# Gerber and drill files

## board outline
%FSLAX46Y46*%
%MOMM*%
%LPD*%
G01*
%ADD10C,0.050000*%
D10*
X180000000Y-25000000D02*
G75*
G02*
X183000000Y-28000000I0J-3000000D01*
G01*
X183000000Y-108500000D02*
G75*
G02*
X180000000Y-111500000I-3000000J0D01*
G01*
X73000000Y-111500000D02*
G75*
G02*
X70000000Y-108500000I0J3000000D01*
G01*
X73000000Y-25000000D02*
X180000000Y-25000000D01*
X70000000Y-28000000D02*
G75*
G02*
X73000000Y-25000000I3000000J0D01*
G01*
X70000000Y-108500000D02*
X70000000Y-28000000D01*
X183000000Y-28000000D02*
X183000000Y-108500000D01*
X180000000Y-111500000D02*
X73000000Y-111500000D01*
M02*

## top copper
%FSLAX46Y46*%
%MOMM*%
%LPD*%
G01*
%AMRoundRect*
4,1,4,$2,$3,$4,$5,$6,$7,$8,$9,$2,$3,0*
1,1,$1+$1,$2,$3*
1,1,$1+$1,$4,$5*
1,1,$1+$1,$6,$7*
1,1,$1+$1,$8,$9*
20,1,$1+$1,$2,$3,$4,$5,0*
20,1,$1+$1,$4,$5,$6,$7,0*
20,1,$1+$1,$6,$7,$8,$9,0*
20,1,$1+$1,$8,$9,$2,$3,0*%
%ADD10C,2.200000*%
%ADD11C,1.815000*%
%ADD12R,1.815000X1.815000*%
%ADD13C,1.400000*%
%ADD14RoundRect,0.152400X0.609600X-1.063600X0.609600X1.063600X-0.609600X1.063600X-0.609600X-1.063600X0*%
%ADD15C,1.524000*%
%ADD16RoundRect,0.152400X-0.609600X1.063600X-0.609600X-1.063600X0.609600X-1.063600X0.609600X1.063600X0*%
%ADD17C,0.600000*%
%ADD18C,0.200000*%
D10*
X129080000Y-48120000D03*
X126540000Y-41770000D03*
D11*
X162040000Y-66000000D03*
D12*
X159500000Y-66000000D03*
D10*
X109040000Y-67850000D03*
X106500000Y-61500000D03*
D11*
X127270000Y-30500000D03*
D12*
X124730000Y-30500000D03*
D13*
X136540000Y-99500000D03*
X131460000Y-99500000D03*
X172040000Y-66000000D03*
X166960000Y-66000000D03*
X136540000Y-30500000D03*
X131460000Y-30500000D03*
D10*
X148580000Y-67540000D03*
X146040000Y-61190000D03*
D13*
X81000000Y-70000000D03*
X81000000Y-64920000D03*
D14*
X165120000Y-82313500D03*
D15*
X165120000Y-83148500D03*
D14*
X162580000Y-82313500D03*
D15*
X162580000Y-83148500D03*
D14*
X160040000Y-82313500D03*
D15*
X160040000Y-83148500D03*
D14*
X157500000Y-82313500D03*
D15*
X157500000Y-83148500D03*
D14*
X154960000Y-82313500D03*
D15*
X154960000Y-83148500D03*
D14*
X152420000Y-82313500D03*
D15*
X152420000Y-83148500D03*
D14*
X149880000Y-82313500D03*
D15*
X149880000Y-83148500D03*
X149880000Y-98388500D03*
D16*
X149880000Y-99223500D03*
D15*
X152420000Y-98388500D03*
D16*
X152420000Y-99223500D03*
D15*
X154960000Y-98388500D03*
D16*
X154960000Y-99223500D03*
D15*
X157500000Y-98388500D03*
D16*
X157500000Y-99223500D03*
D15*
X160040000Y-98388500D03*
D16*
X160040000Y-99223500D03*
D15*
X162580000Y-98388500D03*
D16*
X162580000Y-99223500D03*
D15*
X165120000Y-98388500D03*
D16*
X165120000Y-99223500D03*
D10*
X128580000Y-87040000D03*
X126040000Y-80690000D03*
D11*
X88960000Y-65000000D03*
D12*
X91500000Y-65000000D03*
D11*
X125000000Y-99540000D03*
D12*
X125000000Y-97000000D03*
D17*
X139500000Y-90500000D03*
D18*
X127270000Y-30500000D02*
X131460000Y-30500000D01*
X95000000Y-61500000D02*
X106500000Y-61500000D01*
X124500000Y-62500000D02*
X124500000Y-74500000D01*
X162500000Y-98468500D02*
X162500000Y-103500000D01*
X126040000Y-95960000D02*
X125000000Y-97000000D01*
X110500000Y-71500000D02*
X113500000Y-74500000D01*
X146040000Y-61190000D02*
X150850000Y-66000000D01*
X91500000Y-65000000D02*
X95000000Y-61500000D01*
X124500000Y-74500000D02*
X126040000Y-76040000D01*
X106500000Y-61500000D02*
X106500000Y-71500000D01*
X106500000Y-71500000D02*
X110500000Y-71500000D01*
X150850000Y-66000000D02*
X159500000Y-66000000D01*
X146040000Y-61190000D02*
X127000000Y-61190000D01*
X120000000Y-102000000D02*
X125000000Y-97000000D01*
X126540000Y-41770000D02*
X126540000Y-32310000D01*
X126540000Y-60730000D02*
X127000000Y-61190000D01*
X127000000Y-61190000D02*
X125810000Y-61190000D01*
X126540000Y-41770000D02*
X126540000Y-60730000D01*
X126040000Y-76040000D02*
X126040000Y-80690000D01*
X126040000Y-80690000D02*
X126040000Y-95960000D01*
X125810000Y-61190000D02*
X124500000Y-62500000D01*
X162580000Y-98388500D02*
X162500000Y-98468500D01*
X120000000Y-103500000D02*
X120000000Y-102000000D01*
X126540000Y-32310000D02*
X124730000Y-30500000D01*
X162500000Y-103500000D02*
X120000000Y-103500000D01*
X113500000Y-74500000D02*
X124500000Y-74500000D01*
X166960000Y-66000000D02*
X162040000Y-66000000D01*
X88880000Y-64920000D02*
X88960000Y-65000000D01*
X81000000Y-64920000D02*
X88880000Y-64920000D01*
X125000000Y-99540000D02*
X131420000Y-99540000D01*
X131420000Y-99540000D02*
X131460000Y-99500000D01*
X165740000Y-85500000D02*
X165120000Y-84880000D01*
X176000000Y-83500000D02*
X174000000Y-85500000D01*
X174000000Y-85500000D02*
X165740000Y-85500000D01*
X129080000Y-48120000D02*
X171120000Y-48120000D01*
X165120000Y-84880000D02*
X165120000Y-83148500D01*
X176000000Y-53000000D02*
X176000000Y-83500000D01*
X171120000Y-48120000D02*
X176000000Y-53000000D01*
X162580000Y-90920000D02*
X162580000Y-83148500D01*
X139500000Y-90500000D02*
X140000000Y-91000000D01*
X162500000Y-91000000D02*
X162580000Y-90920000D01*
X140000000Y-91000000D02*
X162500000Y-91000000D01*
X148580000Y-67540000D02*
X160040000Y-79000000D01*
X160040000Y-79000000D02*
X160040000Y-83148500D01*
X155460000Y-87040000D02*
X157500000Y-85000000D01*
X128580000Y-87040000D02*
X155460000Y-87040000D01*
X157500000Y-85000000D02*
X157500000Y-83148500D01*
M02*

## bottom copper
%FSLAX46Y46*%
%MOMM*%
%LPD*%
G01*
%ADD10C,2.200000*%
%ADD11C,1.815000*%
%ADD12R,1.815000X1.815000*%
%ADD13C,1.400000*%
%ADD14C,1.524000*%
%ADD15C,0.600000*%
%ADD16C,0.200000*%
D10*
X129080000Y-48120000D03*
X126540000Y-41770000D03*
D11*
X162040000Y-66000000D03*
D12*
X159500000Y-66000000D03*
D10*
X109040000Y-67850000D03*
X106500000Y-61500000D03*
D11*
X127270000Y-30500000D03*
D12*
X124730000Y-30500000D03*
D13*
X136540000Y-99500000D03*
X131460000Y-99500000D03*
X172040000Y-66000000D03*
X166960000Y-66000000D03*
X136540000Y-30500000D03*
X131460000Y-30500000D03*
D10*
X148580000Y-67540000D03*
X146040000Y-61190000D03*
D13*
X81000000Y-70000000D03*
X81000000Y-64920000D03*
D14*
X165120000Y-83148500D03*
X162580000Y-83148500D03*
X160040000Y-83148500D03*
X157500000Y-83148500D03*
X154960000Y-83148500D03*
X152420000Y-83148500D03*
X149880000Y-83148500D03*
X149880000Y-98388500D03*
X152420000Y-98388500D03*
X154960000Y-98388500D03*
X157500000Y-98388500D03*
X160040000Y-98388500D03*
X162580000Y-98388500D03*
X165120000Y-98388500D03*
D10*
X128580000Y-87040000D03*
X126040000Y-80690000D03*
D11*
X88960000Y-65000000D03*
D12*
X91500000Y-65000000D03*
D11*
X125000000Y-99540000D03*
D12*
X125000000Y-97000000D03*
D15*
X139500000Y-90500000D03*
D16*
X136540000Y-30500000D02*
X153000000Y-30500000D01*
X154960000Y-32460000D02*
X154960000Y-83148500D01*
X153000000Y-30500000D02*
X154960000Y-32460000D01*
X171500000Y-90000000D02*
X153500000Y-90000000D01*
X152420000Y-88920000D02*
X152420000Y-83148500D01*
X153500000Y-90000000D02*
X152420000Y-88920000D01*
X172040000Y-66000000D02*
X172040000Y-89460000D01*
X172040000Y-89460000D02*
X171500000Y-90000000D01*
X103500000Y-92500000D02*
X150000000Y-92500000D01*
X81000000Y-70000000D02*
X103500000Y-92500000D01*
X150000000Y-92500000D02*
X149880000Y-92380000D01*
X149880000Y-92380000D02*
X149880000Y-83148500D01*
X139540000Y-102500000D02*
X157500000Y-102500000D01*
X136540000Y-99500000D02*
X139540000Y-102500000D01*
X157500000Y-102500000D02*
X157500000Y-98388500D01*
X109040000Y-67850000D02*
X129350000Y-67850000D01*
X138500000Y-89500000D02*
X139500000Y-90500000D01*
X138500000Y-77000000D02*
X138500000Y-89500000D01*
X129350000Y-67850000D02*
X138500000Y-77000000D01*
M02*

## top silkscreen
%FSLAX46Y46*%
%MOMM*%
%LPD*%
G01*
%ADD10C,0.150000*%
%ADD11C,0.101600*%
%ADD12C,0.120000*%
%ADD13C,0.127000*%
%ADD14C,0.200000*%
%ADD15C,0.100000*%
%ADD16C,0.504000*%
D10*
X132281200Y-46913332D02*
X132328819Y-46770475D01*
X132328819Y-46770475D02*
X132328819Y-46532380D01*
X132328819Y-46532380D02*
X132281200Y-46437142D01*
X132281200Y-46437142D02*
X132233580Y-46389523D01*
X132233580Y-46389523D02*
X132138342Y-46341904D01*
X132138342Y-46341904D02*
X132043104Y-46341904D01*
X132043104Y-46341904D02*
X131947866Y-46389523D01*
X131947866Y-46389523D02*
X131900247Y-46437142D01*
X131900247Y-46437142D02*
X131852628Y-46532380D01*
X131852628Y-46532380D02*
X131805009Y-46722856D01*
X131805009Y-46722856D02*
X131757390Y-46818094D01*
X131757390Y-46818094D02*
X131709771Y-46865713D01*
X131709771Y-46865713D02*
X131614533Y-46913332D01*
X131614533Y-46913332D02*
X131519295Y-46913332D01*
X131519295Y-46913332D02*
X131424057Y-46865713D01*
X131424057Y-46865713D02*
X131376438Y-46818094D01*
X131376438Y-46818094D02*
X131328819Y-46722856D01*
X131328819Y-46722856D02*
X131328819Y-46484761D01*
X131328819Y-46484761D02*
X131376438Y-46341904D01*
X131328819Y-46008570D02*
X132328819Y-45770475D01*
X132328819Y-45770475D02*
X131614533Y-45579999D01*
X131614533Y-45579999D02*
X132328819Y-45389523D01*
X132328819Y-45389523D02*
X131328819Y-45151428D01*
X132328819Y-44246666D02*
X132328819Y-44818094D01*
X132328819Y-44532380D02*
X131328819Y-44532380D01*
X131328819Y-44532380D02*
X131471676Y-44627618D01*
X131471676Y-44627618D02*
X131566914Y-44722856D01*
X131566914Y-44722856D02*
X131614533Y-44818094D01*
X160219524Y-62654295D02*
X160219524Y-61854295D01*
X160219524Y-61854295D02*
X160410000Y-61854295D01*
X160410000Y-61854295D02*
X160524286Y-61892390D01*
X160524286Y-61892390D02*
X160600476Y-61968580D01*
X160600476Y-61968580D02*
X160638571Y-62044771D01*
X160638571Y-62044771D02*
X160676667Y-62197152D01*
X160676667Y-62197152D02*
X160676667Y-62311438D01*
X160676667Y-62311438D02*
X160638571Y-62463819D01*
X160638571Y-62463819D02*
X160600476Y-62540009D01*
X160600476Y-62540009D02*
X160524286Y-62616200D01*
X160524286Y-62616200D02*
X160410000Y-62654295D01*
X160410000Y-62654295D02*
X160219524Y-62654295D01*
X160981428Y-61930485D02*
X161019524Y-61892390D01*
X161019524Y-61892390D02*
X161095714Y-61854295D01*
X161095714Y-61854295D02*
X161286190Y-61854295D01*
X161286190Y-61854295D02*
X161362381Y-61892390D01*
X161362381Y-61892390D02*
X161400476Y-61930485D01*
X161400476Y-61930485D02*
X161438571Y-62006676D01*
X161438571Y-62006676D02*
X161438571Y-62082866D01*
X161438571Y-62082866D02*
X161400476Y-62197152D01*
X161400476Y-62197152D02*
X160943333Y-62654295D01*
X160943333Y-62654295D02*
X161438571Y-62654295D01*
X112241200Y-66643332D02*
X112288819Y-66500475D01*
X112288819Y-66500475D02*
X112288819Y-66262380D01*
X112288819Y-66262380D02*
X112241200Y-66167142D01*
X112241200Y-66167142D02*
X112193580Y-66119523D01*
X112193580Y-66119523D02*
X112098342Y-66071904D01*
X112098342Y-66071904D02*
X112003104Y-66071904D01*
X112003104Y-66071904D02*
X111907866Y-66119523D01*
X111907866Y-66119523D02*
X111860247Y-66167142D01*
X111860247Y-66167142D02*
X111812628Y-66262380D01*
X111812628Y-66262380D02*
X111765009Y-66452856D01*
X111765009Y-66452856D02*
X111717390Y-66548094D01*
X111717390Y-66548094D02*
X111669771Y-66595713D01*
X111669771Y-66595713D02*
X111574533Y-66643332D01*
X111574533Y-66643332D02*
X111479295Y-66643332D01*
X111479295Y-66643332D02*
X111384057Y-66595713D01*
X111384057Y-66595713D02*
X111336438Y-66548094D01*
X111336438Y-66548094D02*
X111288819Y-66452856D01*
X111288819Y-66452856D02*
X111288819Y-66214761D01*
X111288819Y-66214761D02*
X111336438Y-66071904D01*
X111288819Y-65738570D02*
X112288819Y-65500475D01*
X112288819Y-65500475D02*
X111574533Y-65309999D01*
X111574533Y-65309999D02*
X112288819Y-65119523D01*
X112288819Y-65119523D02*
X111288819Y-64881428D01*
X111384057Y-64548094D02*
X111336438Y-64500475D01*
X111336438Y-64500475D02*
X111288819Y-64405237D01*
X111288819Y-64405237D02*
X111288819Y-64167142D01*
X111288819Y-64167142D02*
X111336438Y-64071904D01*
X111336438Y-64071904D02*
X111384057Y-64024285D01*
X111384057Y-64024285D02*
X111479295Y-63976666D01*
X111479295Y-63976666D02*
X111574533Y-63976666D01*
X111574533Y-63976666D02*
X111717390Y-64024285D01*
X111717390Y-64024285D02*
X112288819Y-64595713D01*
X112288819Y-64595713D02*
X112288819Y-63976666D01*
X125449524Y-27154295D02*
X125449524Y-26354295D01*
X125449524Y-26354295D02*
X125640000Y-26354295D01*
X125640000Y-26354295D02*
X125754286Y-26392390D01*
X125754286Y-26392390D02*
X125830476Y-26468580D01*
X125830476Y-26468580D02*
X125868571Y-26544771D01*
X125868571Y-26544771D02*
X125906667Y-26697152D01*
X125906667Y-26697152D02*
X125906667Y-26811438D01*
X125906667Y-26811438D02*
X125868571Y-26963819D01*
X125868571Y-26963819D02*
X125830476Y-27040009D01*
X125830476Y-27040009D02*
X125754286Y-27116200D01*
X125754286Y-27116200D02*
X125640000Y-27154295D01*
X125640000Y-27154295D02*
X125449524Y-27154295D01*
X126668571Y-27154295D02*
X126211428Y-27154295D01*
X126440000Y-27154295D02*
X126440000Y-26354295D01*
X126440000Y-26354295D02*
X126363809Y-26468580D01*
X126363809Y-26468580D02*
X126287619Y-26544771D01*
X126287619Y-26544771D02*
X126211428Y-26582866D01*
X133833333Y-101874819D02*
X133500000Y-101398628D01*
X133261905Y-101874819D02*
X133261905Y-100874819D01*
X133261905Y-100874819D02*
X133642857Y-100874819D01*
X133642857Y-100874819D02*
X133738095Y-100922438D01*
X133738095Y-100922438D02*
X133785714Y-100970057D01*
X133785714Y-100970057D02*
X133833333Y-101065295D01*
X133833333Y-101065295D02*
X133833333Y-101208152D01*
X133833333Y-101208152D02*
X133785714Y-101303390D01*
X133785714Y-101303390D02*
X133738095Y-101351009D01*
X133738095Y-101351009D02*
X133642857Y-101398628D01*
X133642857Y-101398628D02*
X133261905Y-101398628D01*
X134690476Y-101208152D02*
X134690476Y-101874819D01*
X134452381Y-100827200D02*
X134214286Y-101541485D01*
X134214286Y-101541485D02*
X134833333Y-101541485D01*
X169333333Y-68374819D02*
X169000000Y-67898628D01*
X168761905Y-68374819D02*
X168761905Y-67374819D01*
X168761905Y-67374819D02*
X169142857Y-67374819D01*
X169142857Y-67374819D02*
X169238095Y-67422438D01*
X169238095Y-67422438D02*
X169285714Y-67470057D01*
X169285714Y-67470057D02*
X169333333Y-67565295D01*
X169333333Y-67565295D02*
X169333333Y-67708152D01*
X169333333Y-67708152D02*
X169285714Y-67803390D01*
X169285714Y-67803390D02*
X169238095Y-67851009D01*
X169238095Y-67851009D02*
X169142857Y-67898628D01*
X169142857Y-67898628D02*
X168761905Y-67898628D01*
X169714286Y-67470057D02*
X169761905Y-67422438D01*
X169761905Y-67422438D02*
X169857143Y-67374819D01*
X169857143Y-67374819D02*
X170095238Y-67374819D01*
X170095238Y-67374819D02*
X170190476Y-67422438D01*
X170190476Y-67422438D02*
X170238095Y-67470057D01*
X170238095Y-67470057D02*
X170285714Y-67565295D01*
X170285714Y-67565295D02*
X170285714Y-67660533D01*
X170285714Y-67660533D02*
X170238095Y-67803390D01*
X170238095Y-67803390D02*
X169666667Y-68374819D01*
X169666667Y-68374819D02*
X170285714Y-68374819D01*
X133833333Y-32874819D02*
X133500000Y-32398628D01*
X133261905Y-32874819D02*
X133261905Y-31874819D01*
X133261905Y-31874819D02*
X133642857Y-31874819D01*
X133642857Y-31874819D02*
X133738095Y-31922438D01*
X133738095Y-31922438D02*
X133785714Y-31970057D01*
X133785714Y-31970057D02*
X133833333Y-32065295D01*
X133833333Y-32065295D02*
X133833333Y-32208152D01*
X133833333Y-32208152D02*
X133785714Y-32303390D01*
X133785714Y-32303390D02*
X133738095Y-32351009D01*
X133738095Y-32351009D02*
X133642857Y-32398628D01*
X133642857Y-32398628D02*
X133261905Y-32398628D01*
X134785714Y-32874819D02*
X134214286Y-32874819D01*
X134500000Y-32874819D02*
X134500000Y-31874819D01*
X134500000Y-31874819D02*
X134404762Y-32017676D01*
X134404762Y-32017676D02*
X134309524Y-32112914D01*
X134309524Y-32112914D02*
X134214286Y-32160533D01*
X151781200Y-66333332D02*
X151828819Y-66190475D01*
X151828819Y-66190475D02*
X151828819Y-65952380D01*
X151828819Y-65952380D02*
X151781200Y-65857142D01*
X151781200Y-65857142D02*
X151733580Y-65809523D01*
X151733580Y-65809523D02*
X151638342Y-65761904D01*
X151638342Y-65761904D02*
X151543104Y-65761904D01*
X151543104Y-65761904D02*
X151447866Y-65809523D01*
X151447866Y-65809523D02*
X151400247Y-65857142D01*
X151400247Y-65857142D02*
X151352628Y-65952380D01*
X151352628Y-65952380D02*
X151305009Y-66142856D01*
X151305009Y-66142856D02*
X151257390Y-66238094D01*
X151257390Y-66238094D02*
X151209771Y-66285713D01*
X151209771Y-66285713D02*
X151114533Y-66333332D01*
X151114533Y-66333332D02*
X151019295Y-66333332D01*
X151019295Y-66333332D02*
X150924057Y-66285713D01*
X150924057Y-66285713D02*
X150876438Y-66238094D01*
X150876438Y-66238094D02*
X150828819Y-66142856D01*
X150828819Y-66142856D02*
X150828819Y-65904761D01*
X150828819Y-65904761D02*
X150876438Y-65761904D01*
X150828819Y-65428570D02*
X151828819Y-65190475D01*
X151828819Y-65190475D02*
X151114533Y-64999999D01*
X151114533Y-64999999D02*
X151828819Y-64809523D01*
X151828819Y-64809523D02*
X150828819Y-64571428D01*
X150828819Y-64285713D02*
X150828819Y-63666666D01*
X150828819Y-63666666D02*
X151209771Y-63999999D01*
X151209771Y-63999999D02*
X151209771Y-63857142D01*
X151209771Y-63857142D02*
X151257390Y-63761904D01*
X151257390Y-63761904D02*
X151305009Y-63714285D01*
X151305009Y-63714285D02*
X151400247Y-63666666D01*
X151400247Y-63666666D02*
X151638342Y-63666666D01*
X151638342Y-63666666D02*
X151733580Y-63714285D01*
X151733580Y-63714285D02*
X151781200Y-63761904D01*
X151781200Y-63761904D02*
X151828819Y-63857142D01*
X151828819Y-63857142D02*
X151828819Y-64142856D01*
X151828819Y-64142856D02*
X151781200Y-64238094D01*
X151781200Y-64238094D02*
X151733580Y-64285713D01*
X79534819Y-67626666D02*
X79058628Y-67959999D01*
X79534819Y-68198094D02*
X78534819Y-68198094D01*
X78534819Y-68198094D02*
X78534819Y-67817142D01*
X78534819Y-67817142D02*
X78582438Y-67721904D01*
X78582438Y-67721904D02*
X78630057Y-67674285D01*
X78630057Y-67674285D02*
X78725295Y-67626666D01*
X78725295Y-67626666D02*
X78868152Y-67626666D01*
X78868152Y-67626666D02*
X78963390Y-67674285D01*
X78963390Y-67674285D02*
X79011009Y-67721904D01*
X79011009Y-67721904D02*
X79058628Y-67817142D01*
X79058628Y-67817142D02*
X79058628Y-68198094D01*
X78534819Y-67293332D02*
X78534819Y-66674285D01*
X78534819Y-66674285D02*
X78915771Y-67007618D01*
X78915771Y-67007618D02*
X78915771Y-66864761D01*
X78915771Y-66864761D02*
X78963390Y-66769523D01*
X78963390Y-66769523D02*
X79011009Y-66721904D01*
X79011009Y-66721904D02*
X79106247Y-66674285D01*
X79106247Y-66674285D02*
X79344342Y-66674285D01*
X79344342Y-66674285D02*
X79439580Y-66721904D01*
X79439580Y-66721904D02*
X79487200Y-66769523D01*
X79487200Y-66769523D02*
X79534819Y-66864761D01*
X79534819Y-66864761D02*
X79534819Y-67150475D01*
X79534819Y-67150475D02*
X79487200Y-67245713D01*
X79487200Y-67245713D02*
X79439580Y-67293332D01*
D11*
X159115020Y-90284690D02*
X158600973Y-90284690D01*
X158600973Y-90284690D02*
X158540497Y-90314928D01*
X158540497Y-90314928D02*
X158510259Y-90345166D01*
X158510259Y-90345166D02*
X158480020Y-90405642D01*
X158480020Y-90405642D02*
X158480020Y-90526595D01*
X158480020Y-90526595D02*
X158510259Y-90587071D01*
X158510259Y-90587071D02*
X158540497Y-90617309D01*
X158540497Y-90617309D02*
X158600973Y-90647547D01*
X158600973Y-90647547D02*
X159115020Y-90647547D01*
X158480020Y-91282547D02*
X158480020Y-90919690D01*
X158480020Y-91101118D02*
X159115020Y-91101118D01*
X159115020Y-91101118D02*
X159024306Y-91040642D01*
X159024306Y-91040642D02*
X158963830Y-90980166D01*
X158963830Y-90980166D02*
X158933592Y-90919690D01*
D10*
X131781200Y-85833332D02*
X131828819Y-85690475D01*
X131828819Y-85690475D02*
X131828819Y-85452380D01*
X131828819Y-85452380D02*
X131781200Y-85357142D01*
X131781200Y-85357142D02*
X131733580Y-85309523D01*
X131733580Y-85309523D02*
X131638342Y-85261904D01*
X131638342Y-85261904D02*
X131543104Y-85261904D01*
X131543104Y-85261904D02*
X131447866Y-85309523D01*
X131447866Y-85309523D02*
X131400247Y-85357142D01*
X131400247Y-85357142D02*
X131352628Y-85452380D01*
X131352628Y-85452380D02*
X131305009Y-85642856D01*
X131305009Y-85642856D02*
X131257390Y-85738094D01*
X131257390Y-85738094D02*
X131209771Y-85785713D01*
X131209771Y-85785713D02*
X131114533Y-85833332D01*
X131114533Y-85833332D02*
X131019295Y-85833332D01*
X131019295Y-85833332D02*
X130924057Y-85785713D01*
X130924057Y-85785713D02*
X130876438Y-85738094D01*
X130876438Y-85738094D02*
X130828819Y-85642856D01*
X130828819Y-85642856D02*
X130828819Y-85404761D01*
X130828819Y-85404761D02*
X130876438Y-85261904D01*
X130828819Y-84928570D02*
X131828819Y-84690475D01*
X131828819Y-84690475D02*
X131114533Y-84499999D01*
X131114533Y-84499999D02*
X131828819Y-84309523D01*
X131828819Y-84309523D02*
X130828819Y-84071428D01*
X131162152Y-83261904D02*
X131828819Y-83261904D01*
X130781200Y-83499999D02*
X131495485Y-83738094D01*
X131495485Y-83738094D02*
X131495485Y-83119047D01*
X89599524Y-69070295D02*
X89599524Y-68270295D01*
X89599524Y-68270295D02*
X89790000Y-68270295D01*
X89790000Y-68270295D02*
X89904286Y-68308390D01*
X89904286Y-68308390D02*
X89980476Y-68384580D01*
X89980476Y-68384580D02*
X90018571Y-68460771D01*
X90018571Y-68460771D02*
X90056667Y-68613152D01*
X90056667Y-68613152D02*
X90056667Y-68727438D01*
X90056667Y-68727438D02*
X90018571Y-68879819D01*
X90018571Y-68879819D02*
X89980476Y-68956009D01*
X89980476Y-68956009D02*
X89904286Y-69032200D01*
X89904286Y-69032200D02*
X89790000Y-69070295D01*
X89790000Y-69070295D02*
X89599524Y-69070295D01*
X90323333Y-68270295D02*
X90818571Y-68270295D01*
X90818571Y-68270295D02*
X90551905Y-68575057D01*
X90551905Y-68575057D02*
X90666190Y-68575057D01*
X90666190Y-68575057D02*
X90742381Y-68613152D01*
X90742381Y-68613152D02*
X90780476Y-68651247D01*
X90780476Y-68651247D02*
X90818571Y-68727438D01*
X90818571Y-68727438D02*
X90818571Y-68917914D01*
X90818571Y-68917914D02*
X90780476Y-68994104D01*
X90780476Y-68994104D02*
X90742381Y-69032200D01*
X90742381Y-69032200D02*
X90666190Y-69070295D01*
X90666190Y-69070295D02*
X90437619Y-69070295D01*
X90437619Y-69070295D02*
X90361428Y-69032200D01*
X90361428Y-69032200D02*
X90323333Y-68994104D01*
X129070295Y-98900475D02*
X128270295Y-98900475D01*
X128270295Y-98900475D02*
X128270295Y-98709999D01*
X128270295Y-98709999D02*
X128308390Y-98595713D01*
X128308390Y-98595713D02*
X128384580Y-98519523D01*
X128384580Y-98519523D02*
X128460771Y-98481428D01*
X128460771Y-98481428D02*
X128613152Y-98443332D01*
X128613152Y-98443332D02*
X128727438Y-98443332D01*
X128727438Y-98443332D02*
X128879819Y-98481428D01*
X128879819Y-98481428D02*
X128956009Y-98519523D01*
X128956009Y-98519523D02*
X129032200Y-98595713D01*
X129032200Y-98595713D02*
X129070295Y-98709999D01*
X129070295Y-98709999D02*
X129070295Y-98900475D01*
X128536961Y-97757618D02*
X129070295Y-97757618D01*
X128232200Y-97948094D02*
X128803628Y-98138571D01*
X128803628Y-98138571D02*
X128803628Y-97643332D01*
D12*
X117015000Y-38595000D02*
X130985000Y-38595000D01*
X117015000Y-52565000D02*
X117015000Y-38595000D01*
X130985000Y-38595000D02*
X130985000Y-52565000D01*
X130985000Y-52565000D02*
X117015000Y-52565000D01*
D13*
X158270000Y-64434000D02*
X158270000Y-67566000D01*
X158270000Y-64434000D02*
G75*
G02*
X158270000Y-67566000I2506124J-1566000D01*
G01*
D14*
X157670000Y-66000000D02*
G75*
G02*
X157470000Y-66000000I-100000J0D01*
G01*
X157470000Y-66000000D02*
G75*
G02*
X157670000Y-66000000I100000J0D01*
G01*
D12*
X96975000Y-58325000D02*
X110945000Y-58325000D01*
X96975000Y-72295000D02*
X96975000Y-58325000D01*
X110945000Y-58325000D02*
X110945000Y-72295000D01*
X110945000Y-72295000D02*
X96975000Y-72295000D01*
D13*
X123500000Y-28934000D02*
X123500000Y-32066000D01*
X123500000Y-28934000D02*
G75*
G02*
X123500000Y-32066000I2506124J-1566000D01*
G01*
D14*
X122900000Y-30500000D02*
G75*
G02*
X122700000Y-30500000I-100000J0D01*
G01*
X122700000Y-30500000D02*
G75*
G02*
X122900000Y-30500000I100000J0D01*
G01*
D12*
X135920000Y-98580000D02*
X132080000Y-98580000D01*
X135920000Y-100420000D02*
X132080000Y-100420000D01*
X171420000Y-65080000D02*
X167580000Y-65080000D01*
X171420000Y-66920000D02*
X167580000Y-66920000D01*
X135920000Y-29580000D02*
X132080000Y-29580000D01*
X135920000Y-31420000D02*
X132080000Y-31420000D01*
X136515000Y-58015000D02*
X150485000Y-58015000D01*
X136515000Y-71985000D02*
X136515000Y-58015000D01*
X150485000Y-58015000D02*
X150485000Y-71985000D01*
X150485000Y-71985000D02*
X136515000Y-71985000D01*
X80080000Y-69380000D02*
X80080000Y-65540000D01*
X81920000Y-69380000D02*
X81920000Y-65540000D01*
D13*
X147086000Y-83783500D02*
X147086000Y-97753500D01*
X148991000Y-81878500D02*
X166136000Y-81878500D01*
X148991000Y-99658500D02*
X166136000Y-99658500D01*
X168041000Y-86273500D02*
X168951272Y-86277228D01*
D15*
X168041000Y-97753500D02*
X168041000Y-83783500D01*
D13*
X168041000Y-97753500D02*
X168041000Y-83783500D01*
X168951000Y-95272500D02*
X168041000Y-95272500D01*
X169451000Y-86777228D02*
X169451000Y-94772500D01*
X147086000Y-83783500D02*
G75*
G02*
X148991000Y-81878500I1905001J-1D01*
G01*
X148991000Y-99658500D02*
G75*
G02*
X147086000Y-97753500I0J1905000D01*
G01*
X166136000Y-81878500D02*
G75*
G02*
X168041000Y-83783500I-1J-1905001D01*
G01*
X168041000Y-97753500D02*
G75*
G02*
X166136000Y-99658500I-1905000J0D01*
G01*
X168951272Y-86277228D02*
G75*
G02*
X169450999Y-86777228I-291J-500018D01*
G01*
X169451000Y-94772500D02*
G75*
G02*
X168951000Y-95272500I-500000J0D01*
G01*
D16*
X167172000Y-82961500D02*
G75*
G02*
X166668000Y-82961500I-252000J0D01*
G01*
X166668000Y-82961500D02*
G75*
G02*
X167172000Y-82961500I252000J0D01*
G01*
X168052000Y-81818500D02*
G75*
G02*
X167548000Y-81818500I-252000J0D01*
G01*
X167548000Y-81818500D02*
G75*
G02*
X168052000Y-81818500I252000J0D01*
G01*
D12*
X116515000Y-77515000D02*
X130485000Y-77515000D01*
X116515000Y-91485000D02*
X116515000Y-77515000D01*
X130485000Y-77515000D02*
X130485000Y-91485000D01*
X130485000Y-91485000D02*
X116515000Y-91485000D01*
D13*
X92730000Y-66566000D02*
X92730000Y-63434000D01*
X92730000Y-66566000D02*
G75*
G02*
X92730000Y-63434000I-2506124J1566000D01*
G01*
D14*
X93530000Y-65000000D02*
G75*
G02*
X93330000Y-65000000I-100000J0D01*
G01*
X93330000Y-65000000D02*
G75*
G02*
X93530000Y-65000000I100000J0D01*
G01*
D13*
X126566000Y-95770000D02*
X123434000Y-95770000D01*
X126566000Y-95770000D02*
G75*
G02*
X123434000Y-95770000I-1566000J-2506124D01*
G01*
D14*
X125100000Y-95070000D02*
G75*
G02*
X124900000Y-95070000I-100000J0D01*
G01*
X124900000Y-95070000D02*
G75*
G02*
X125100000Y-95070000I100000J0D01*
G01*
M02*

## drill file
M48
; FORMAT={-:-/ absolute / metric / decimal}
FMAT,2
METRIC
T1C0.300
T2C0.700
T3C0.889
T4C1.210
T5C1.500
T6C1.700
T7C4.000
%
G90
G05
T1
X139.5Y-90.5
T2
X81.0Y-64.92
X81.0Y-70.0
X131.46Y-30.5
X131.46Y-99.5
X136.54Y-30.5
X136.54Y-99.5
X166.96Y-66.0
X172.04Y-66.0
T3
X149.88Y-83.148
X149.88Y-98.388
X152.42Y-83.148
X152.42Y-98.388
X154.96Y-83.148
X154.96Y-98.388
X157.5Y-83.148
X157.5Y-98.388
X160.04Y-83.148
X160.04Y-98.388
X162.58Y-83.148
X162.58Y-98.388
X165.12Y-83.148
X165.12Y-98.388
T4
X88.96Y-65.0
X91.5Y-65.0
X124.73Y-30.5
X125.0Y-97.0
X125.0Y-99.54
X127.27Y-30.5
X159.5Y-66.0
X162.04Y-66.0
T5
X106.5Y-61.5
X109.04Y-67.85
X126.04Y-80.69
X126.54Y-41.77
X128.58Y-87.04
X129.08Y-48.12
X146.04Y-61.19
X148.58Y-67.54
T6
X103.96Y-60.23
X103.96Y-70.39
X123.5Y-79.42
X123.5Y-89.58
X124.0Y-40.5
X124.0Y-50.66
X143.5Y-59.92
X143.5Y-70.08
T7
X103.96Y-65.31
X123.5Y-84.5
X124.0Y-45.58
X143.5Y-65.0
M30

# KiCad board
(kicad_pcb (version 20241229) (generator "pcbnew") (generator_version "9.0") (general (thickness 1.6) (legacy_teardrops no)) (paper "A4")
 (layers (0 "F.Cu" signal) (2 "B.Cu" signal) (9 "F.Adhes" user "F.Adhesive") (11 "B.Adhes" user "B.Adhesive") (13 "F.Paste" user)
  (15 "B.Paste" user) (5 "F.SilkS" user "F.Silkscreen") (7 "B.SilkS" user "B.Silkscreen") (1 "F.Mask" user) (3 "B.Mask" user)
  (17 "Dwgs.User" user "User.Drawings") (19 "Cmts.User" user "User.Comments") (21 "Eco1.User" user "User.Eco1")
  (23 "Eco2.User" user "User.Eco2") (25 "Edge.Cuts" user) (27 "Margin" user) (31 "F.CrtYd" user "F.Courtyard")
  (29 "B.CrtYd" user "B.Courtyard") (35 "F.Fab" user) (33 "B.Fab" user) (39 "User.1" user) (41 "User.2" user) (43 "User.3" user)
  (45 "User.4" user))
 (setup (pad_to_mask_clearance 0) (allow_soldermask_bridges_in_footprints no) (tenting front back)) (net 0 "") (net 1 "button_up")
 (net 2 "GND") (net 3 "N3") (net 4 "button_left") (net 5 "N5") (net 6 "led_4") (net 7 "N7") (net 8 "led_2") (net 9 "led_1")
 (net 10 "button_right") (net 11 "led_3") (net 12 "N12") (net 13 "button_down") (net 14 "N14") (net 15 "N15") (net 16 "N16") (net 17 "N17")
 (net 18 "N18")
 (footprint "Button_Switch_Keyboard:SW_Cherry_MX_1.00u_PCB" (layer "F.Cu") (at 129.08 48.12 -90)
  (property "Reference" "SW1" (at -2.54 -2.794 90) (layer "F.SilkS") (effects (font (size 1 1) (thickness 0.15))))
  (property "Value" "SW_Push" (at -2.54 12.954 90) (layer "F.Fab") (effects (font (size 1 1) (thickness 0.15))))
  (fp_line (start -9.525 12.065) (end -9.525 -1.905) (stroke (width 0.12) (type solid)) (layer "F.SilkS"))
  (fp_line (start 4.445 12.065) (end -9.525 12.065) (stroke (width 0.12) (type solid)) (layer "F.SilkS"))
  (fp_line (start -9.525 -1.905) (end 4.445 -1.905) (stroke (width 0.12) (type solid)) (layer "F.SilkS"))
  (fp_line (start 4.445 -1.905) (end 4.445 12.065) (stroke (width 0.12) (type solid)) (layer "F.SilkS"))
  (pad "" np_thru_hole circle (at -7.62 5.08 270) (size 1.7 1.7) (drill 1.7) (layers "*.Cu" "*.Mask"))
  (pad "" np_thru_hole circle (at -2.54 5.08 270) (size 4 4) (drill 4) (layers "*.Cu" "*.Mask"))
  (pad "" np_thru_hole circle (at 2.54 5.08 270) (size 1.7 1.7) (drill 1.7) (layers "*.Cu" "*.Mask"))
  (pad "1" thru_hole circle (at 0 0 270) (size 2.2 2.2) (drill 1.5) (layers "*.Cu" "*.Mask") (remove_unused_layers no) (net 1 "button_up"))
  (pad "2" thru_hole circle (at -6.35 2.54 270) (size 2.2 2.2) (drill 1.5) (layers "*.Cu" "*.Mask") (remove_unused_layers no) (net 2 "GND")))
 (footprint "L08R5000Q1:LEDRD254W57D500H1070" (layer "F.Cu") (at 160.77 66)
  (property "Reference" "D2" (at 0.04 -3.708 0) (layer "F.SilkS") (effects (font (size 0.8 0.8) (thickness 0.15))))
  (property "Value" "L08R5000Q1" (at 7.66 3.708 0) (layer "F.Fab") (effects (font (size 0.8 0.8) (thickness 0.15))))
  (fp_line (start -2.5 -1.566) (end -2.5 1.566) (stroke (width 0.127) (type solid)) (layer "F.SilkS"))
  (fp_arc (start -2.5 -1.566) (mid 2.961291 0) (end -2.5 1.566) (stroke (width 0.127) (type solid)) (layer "F.SilkS"))
  (fp_circle (center -3.2 0) (end -3.1 0) (stroke (width 0.2) (type solid)) (fill no) (layer "F.SilkS"))
  (pad "A" thru_hole circle (at 1.27 0) (size 1.815 1.815) (drill 1.21) (layers "*.Cu" "*.Mask") (remove_unused_layers no) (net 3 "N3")
   (solder_mask_margin 0.102))
  (pad "C" thru_hole rect (at -1.27 0) (size 1.815 1.815) (drill 1.21) (layers "*.Cu" "*.Mask") (remove_unused_layers no) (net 2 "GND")
   (solder_mask_margin 0.102)))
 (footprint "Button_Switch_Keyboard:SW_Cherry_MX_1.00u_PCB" (layer "F.Cu") (at 109.04 67.85 -90)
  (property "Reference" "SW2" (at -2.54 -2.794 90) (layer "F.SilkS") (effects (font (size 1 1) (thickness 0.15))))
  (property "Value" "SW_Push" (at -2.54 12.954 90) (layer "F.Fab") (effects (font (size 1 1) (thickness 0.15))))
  (fp_line (start -9.525 12.065) (end -9.525 -1.905) (stroke (width 0.12) (type solid)) (layer "F.SilkS"))
  (fp_line (start 4.445 12.065) (end -9.525 12.065) (stroke (width 0.12) (type solid)) (layer "F.SilkS"))
  (fp_line (start -9.525 -1.905) (end 4.445 -1.905) (stroke (width 0.12) (type solid)) (layer "F.SilkS"))
  (fp_line (start 4.445 -1.905) (end 4.445 12.065) (stroke (width 0.12) (type solid)) (layer "F.SilkS"))
  (pad "" np_thru_hole circle (at -7.62 5.08 270) (size 1.7 1.7) (drill 1.7) (layers "*.Cu" "*.Mask"))
  (pad "" np_thru_hole circle (at -2.54 5.08 270) (size 4 4) (drill 4) (layers "*.Cu" "*.Mask"))
  (pad "" np_thru_hole circle (at 2.54 5.08 270) (size 1.7 1.7) (drill 1.7) (layers "*.Cu" "*.Mask"))
  (pad "1" thru_hole circle (at 0 0 270) (size 2.2 2.2) (drill 1.5) (layers "*.Cu" "*.Mask") (remove_unused_layers no) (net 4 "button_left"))
  (pad "2" thru_hole circle (at -6.35 2.54 270) (size 2.2 2.2) (drill 1.5) (layers "*.Cu" "*.Mask") (remove_unused_layers no) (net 2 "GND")))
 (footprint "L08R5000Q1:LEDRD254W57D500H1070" (layer "F.Cu") (at 126 30.5)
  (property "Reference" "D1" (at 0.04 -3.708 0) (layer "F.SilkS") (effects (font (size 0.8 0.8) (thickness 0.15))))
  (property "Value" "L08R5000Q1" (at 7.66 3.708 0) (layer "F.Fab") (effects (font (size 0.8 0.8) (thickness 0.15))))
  (fp_line (start -2.5 -1.566) (end -2.5 1.566) (stroke (width 0.127) (type solid)) (layer "F.SilkS"))
  (fp_arc (start -2.5 -1.566) (mid 2.961291 0) (end -2.5 1.566) (stroke (width 0.127) (type solid)) (layer "F.SilkS"))
  (fp_circle (center -3.2 0) (end -3.1 0) (stroke (width 0.2) (type solid)) (fill no) (layer "F.SilkS"))
  (pad "A" thru_hole circle (at 1.27 0) (size 1.815 1.815) (drill 1.21) (layers "*.Cu" "*.Mask") (remove_unused_layers no) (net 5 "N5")
   (solder_mask_margin 0.102))
  (pad "C" thru_hole rect (at -1.27 0) (size 1.815 1.815) (drill 1.21) (layers "*.Cu" "*.Mask") (remove_unused_layers no) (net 2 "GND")
   (solder_mask_margin 0.102)))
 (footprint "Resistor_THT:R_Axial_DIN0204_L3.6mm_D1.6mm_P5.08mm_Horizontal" (layer "F.Cu") (at 136.54 99.5 180)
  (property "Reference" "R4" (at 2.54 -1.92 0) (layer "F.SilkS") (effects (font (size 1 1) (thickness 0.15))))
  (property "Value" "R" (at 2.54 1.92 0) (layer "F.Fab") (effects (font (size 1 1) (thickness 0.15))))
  (fp_line (start 0.62 0.92) (end 4.46 0.92) (stroke (width 0.12) (type solid)) (layer "F.SilkS"))
  (fp_line (start 0.62 -0.92) (end 4.46 -0.92) (stroke (width 0.12) (type solid)) (layer "F.SilkS"))
  (pad "1" thru_hole circle (at 0 0 180) (size 1.4 1.4) (drill 0.7) (layers "*.Cu" "*.Mask") (remove_unused_layers no) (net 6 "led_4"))
  (pad "2" thru_hole circle (at 5.08 0 180) (size 1.4 1.4) (drill 0.7) (layers "*.Cu" "*.Mask") (remove_unused_layers no) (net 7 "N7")))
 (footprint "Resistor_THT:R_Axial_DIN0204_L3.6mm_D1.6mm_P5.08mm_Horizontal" (layer "F.Cu") (at 172.04 66 180)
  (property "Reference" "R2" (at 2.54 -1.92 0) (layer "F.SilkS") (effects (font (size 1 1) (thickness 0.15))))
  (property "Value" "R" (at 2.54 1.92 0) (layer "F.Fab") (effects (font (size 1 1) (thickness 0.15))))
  (fp_line (start 0.62 0.92) (end 4.46 0.92) (stroke (width 0.12) (type solid)) (layer "F.SilkS"))
  (fp_line (start 0.62 -0.92) (end 4.46 -0.92) (stroke (width 0.12) (type solid)) (layer "F.SilkS"))
  (pad "1" thru_hole circle (at 0 0 180) (size 1.4 1.4) (drill 0.7) (layers "*.Cu" "*.Mask") (remove_unused_layers no) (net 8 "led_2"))
  (pad "2" thru_hole circle (at 5.08 0 180) (size 1.4 1.4) (drill 0.7) (layers "*.Cu" "*.Mask") (remove_unused_layers no) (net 3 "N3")))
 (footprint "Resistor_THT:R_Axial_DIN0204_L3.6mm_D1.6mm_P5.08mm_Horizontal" (layer "F.Cu") (at 136.54 30.5 180)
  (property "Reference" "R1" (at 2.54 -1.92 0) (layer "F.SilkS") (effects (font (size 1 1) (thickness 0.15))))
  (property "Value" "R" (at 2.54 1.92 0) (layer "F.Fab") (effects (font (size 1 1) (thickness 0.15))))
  (fp_line (start 0.62 0.92) (end 4.46 0.92) (stroke (width 0.12) (type solid)) (layer "F.SilkS"))
  (fp_line (start 0.62 -0.92) (end 4.46 -0.92) (stroke (width 0.12) (type solid)) (layer "F.SilkS"))
  (pad "1" thru_hole circle (at 0 0 180) (size 1.4 1.4) (drill 0.7) (layers "*.Cu" "*.Mask") (remove_unused_layers no) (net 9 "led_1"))
  (pad "2" thru_hole circle (at 5.08 0 180) (size 1.4 1.4) (drill 0.7) (layers "*.Cu" "*.Mask") (remove_unused_layers no) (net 5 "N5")))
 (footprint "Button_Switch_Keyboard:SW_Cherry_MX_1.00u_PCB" (layer "F.Cu") (at 148.58 67.54 -90)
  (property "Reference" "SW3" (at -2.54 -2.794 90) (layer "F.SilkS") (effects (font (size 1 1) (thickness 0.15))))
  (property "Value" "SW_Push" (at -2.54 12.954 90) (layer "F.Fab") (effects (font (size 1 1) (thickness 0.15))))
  (fp_line (start -9.525 12.065) (end -9.525 -1.905) (stroke (width 0.12) (type solid)) (layer "F.SilkS"))
  (fp_line (start 4.445 12.065) (end -9.525 12.065) (stroke (width 0.12) (type solid)) (layer "F.SilkS"))
  (fp_line (start -9.525 -1.905) (end 4.445 -1.905) (stroke (width 0.12) (type solid)) (layer "F.SilkS"))
  (fp_line (start 4.445 -1.905) (end 4.445 12.065) (stroke (width 0.12) (type solid)) (layer "F.SilkS"))
  (pad "" np_thru_hole circle (at -7.62 5.08 270) (size 1.7 1.7) (drill 1.7) (layers "*.Cu" "*.Mask"))
  (pad "" np_thru_hole circle (at -2.54 5.08 270) (size 4 4) (drill 4) (layers "*.Cu" "*.Mask"))
  (pad "" np_thru_hole circle (at 2.54 5.08 270) (size 1.7 1.7) (drill 1.7) (layers "*.Cu" "*.Mask"))
  (pad "1" thru_hole circle (at 0 0 270) (size 2.2 2.2) (drill 1.5) (layers "*.Cu" "*.Mask") (remove_unused_layers no)
   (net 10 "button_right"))
  (pad "2" thru_hole circle (at -6.35 2.54 270) (size 2.2 2.2) (drill 1.5) (layers "*.Cu" "*.Mask") (remove_unused_layers no) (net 2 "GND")))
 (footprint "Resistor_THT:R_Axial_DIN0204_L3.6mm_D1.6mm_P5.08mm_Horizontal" (layer "F.Cu") (at 81 70 90)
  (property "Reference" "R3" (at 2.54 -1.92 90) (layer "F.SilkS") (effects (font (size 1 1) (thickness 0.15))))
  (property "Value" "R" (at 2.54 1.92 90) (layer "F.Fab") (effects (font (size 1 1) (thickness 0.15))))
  (fp_line (start 0.62 -0.92) (end 4.46 -0.92) (stroke (width 0.12) (type solid)) (layer "F.SilkS"))
  (fp_line (start 0.62 0.92) (end 4.46 0.92) (stroke (width 0.12) (type solid)) (layer "F.SilkS"))
  (pad "1" thru_hole circle (at 0 0 90) (size 1.4 1.4) (drill 0.7) (layers "*.Cu" "*.Mask") (remove_unused_layers no) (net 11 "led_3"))
  (pad "2" thru_hole circle (at 5.08 0 90) (size 1.4 1.4) (drill 0.7) (layers "*.Cu" "*.Mask") (remove_unused_layers no) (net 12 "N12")))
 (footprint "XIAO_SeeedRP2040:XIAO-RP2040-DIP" (layer "F.Cu") (at 157.5 90.7685 -90)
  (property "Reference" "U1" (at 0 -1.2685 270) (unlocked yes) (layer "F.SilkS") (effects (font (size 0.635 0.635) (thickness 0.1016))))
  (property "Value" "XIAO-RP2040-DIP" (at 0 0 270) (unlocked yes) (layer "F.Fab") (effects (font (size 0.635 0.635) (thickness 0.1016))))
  (fp_line (start -6.985 10.414) (end 6.985 10.414) (stroke (width 0.127) (type solid)) (layer "F.SilkS"))
  (fp_line (start -8.89 8.509) (end -8.89 -8.636) (stroke (width 0.127) (type solid)) (layer "F.SilkS"))
  (fp_line (start 8.89 8.509) (end 8.89 -8.636) (stroke (width 0.127) (type solid)) (layer "F.SilkS"))
  (fp_line (start -4.495 -10.541) (end -4.491272 -11.451272) (stroke (width 0.127) (type solid)) (layer "F.SilkS"))
  (fp_line (start 6.985 -10.541) (end -6.985 -10.541) (stroke (width 0.1) (type solid)) (layer "F.SilkS"))
  (fp_line (start 6.985 -10.541) (end -6.985 -10.541) (stroke (width 0.127) (type solid)) (layer "F.SilkS"))
  (fp_line (start 4.504 -11.451) (end 4.504 -10.541) (stroke (width 0.127) (type solid)) (layer "F.SilkS"))
  (fp_line (start -3.991272 -11.951) (end 4.004 -11.951) (stroke (width 0.127) (type solid)) (layer "F.SilkS"))
  (fp_arc (start -6.985 10.414) (mid -8.332038 9.856038) (end -8.89 8.509) (stroke (width 0.127) (type solid)) (layer "F.SilkS"))
  (fp_arc (start 8.89 8.509) (mid 8.332038 9.856038) (end 6.985 10.414) (stroke (width 0.127) (type solid)) (layer "F.SilkS"))
  (fp_arc (start -8.89 -8.636) (mid -8.332038 -9.983038) (end -6.985 -10.541) (stroke (width 0.127) (type solid)) (layer "F.SilkS"))
  (fp_arc (start 6.985 -10.541) (mid 8.332038 -9.983038) (end 8.89 -8.636) (stroke (width 0.127) (type solid)) (layer "F.SilkS"))
  (fp_arc (start -4.491272 -11.451272) (mid -4.344728 -11.80464) (end -3.991272 -11.951) (stroke (width 0.127) (type default))
   (layer "F.SilkS"))
  (fp_arc (start 4.004 -11.951) (mid 4.357553 -11.804553) (end 4.504 -11.451) (stroke (width 0.127) (type default)) (layer "F.SilkS"))
  (fp_circle (center -7.807 -9.42) (end -7.807 -9.674) (stroke (width 0.5) (type solid)) (fill yes) (layer "F.SilkS"))
  (fp_circle (center -8.95 -10.3) (end -8.95 -10.554) (stroke (width 0.5) (type solid)) (fill yes) (layer "F.SilkS"))
  (pad "1" smd roundrect (at -8.455 -7.62 90) (size 2.432 1.524) (layers "F.Cu" "F.Mask") (roundrect_rratio 0.1) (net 1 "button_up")
   (thermal_bridge_angle 45))
  (pad "1" thru_hole circle (at -7.62 -7.62 90) (size 1.524 1.524) (drill 0.889) (layers "*.Cu" "*.Mask") (remove_unused_layers no)
   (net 1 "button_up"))
  (pad "2" smd roundrect (at -8.455 -5.08 90) (size 2.432 1.524) (layers "F.Cu" "F.Mask") (roundrect_rratio 0.1) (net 4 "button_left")
   (thermal_bridge_angle 45))
  (pad "2" thru_hole circle (at -7.62 -5.08 90) (size 1.524 1.524) (drill 0.889) (layers "*.Cu" "*.Mask") (remove_unused_layers no)
   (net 4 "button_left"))
  (pad "3" smd roundrect (at -8.455 -2.54 90) (size 2.432 1.524) (layers "F.Cu" "F.Mask") (roundrect_rratio 0.1) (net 10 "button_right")
   (thermal_bridge_angle 45))
  (pad "3" thru_hole circle (at -7.62 -2.54 90) (size 1.524 1.524) (drill 0.889) (layers "*.Cu" "*.Mask") (remove_unused_layers no)
   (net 10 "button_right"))
  (pad "4" smd roundrect (at -8.455 0 90) (size 2.432 1.524) (layers "F.Cu" "F.Mask") (roundrect_rratio 0.1) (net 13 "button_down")
   (thermal_bridge_angle 45))
  (pad "4" thru_hole circle (at -7.62 0 90) (size 1.524 1.524) (drill 0.889) (layers "*.Cu" "*.Mask") (remove_unused_layers no)
   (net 13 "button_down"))
  (pad "5" smd roundrect (at -8.455 2.54 90) (size 2.432 1.524) (layers "F.Cu" "F.Mask") (roundrect_rratio 0.1) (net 9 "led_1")
   (thermal_bridge_angle 45))
  (pad "5" thru_hole circle (at -7.62 2.54 90) (size 1.524 1.524) (drill 0.889) (layers "*.Cu" "*.Mask") (remove_unused_layers no)
   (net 9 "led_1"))
  (pad "6" smd roundrect (at -8.455 5.08 90) (size 2.432 1.524) (layers "F.Cu" "F.Mask") (roundrect_rratio 0.1) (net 8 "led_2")
   (thermal_bridge_angle 45))
  (pad "6" thru_hole circle (at -7.62 5.08 90) (size 1.524 1.524) (drill 0.889) (layers "*.Cu" "*.Mask") (remove_unused_layers no)
   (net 8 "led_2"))
  (pad "7" smd roundrect (at -8.455 7.62 90) (size 2.432 1.524) (layers "F.Cu" "F.Mask") (roundrect_rratio 0.1) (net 11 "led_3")
   (thermal_bridge_angle 45))
  (pad "7" thru_hole circle (at -7.62 7.62 90) (size 1.524 1.524) (drill 0.889) (layers "*.Cu" "*.Mask") (remove_unused_layers no)
   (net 11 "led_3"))
  (pad "8" thru_hole circle (at 7.62 7.62 270) (size 1.524 1.524) (drill 0.889) (layers "*.Cu" "*.Mask") (remove_unused_layers no)
   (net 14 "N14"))
  (pad "8" smd roundrect (at 8.455 7.62 270) (size 2.432 1.524) (layers "F.Cu" "F.Mask") (roundrect_rratio 0.1) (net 14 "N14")
   (thermal_bridge_angle 45))
  (pad "9" thru_hole circle (at 7.62 5.08 270) (size 1.524 1.524) (drill 0.889) (layers "*.Cu" "*.Mask") (remove_unused_layers no)
   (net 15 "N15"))
  (pad "9" smd roundrect (at 8.455 5.08 270) (size 2.432 1.524) (layers "F.Cu" "F.Mask") (roundrect_rratio 0.1) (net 15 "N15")
   (thermal_bridge_angle 45))
  (pad "10" thru_hole circle (at 7.62 2.54 270) (size 1.524 1.524) (drill 0.889) (layers "*.Cu" "*.Mask") (remove_unused_layers no)
   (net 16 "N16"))
  (pad "10" smd roundrect (at 8.455 2.54 270) (size 2.432 1.524) (layers "F.Cu" "F.Mask") (roundrect_rratio 0.1) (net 16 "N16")
   (thermal_bridge_angle 45))
  (pad "11" thru_hole circle (at 7.62 0 270) (size 1.524 1.524) (drill 0.889) (layers "*.Cu" "*.Mask") (remove_unused_layers no)
   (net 6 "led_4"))
  (pad "11" smd roundrect (at 8.455 0 270) (size 2.432 1.524) (layers "F.Cu" "F.Mask") (roundrect_rratio 0.1) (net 6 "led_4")
   (thermal_bridge_angle 45))
  (pad "12" thru_hole circle (at 7.62 -2.54 270) (size 1.524 1.524) (drill 0.889) (layers "*.Cu" "*.Mask") (remove_unused_layers no)
   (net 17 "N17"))
  (pad "12" smd roundrect (at 8.455 -2.54 270) (size 2.432 1.524) (layers "F.Cu" "F.Mask") (roundrect_rratio 0.1) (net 17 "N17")
   (thermal_bridge_angle 45))
  (pad "13" thru_hole circle (at 7.62 -5.08 270) (size 1.524 1.524) (drill 0.889) (layers "*.Cu" "*.Mask") (remove_unused_layers no)
   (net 2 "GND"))
  (pad "13" smd roundrect (at 8.455 -5.08 270) (size 2.432 1.524) (layers "F.Cu" "F.Mask") (roundrect_rratio 0.1) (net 2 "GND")
   (thermal_bridge_angle 45))
  (pad "14" thru_hole circle (at 7.62 -7.62 270) (size 1.524 1.524) (drill 0.889) (layers "*.Cu" "*.Mask") (remove_unused_layers no)
   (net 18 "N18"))
  (pad "14" smd roundrect (at 8.455 -7.62 270) (size 2.432 1.524) (layers "F.Cu" "F.Mask") (roundrect_rratio 0.1) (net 18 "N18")
   (thermal_bridge_angle 45)))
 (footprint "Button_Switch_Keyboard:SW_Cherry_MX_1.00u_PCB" (layer "F.Cu") (at 128.58 87.04 -90)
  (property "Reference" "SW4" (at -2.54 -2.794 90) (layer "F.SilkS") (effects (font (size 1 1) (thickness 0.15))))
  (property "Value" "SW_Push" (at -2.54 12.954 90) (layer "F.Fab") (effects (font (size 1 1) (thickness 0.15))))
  (fp_line (start -9.525 12.065) (end -9.525 -1.905) (stroke (width 0.12) (type solid)) (layer "F.SilkS"))
  (fp_line (start 4.445 12.065) (end -9.525 12.065) (stroke (width 0.12) (type solid)) (layer "F.SilkS"))
  (fp_line (start -9.525 -1.905) (end 4.445 -1.905) (stroke (width 0.12) (type solid)) (layer "F.SilkS"))
  (fp_line (start 4.445 -1.905) (end 4.445 12.065) (stroke (width 0.12) (type solid)) (layer "F.SilkS"))
  (pad "" np_thru_hole circle (at -7.62 5.08 270) (size 1.7 1.7) (drill 1.7) (layers "*.Cu" "*.Mask"))
  (pad "" np_thru_hole circle (at -2.54 5.08 270) (size 4 4) (drill 4) (layers "*.Cu" "*.Mask"))
  (pad "" np_thru_hole circle (at 2.54 5.08 270) (size 1.7 1.7) (drill 1.7) (layers "*.Cu" "*.Mask"))
  (pad "1" thru_hole circle (at 0 0 270) (size 2.2 2.2) (drill 1.5) (layers "*.Cu" "*.Mask") (remove_unused_layers no)
   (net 13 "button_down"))
  (pad "2" thru_hole circle (at -6.35 2.54 270) (size 2.2 2.2) (drill 1.5) (layers "*.Cu" "*.Mask") (remove_unused_layers no) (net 2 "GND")))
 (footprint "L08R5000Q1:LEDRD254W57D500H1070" (layer "F.Cu") (at 90.23 65 180)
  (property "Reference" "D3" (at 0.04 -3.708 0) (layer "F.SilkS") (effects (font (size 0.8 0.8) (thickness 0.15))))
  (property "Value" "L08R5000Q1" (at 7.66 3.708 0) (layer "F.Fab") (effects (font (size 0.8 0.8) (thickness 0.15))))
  (fp_line (start -2.5 -1.566) (end -2.5 1.566) (stroke (width 0.127) (type solid)) (layer "F.SilkS"))
  (fp_arc (start -2.5 -1.566) (mid 2.961291 0) (end -2.5 1.566) (stroke (width 0.127) (type solid)) (layer "F.SilkS"))
  (fp_circle (center -3.2 0) (end -3.1 0) (stroke (width 0.2) (type solid)) (fill no) (layer "F.SilkS"))
  (pad "A" thru_hole circle (at 1.27 0 180) (size 1.815 1.815) (drill 1.21) (layers "*.Cu" "*.Mask") (remove_unused_layers no)
   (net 12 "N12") (solder_mask_margin 0.102))
  (pad "C" thru_hole rect (at -1.27 0 180) (size 1.815 1.815) (drill 1.21) (layers "*.Cu" "*.Mask") (remove_unused_layers no) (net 2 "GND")
   (solder_mask_margin 0.102)))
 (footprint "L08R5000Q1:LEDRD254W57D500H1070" (layer "F.Cu") (at 125 98.27 -90)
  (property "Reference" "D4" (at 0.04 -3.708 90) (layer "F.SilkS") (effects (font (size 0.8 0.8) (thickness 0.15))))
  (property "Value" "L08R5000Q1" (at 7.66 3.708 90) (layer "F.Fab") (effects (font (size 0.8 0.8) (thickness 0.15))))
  (fp_line (start -2.5 -1.566) (end -2.5 1.566) (stroke (width 0.127) (type solid)) (layer "F.SilkS"))
  (fp_arc (start -2.5 -1.566) (mid 2.961291 0) (end -2.5 1.566) (stroke (width 0.127) (type solid)) (layer "F.SilkS"))
  (fp_circle (center -3.2 0) (end -3.1 0) (stroke (width 0.2) (type solid)) (fill no) (layer "F.SilkS"))
  (pad "A" thru_hole circle (at 1.27 0 270) (size 1.815 1.815) (drill 1.21) (layers "*.Cu" "*.Mask") (remove_unused_layers no) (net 7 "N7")
   (solder_mask_margin 0.102))
  (pad "C" thru_hole rect (at -1.27 0 270) (size 1.815 1.815) (drill 1.21) (layers "*.Cu" "*.Mask") (remove_unused_layers no) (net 2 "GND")
   (solder_mask_margin 0.102)))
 (gr_arc (start 180 25) (mid 182.12132 25.87868) (end 183 28) (stroke (width 0.05) (type default)) (layer "Edge.Cuts"))
 (gr_arc (start 183 108.5) (mid 182.12132 110.62132) (end 180 111.5) (stroke (width 0.05) (type default)) (layer "Edge.Cuts"))
 (gr_arc (start 73 111.5) (mid 70.87868 110.62132) (end 70 108.5) (stroke (width 0.05) (type default)) (layer "Edge.Cuts"))
 (gr_line (start 73 25) (end 180 25) (stroke (width 0.05) (type default)) (layer "Edge.Cuts"))
 (gr_arc (start 70 28) (mid 70.87868 25.87868) (end 73 25) (stroke (width 0.05) (type default)) (layer "Edge.Cuts"))
 (gr_line (start 70 108.5) (end 70 28) (stroke (width 0.05) (type default)) (layer "Edge.Cuts"))
 (gr_line (start 183 28) (end 183 108.5) (stroke (width 0.05) (type default)) (layer "Edge.Cuts"))
 (gr_line (start 180 111.5) (end 73 111.5) (stroke (width 0.05) (type default)) (layer "Edge.Cuts"))
 (segment (start 127.27 30.5) (end 131.46 30.5) (width 0.2) (layer "F.Cu") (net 5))
 (segment (start 95 61.5) (end 106.5 61.5) (width 0.2) (layer "F.Cu") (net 2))
 (segment (start 124.5 62.5) (end 124.5 74.5) (width 0.2) (layer "F.Cu") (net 2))
 (segment (start 162.5 98.4685) (end 162.5 103.5) (width 0.2) (layer "F.Cu") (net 2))
 (segment (start 126.04 95.96) (end 125 97) (width 0.2) (layer "F.Cu") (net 2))
 (segment (start 110.5 71.5) (end 113.5 74.5) (width 0.2) (layer "F.Cu") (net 2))
 (segment (start 146.04 61.19) (end 150.85 66) (width 0.2) (layer "F.Cu") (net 2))
 (segment (start 91.5 65) (end 95 61.5) (width 0.2) (layer "F.Cu") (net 2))
 (segment (start 124.5 74.5) (end 126.04 76.04) (width 0.2) (layer "F.Cu") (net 2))
 (segment (start 106.5 61.5) (end 106.5 71.5) (width 0.2) (layer "F.Cu") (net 2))
 (segment (start 106.5 71.5) (end 110.5 71.5) (width 0.2) (layer "F.Cu") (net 2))
 (segment (start 150.85 66) (end 159.5 66) (width 0.2) (layer "F.Cu") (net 2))
 (segment (start 146.04 61.19) (end 127 61.19) (width 0.2) (layer "F.Cu") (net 2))
 (segment (start 120 102) (end 125 97) (width 0.2) (layer "F.Cu") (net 2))
 (segment (start 126.54 41.77) (end 126.54 32.31) (width 0.2) (layer "F.Cu") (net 2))
 (segment (start 126.54 60.73) (end 127 61.19) (width 0.2) (layer "F.Cu") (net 2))
 (segment (start 127 61.19) (end 125.81 61.19) (width 0.2) (layer "F.Cu") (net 2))
 (segment (start 126.54 41.77) (end 126.54 60.73) (width 0.2) (layer "F.Cu") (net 2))
 (segment (start 126.04 76.04) (end 126.04 80.69) (width 0.2) (layer "F.Cu") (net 2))
 (segment (start 126.04 80.69) (end 126.04 95.96) (width 0.2) (layer "F.Cu") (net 2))
 (segment (start 125.81 61.19) (end 124.5 62.5) (width 0.2) (layer "F.Cu") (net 2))
 (segment (start 162.58 98.3885) (end 162.5 98.4685) (width 0.2) (layer "F.Cu") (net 2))
 (segment (start 120 103.5) (end 120 102) (width 0.2) (layer "F.Cu") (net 2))
 (segment (start 126.54 32.31) (end 124.73 30.5) (width 0.2) (layer "F.Cu") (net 2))
 (segment (start 162.5 103.5) (end 120 103.5) (width 0.2) (layer "F.Cu") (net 2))
 (segment (start 113.5 74.5) (end 124.5 74.5) (width 0.2) (layer "F.Cu") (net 2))
 (segment (start 166.96 66) (end 162.04 66) (width 0.2) (layer "F.Cu") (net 3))
 (segment (start 88.88 64.92) (end 88.96 65) (width 0.2) (layer "F.Cu") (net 12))
 (segment (start 81 64.92) (end 88.88 64.92) (width 0.2) (layer "F.Cu") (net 12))
 (segment (start 125 99.54) (end 131.42 99.54) (width 0.2) (layer "F.Cu") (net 7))
 (segment (start 131.42 99.54) (end 131.46 99.5) (width 0.2) (layer "F.Cu") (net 7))
 (segment (start 136.54 30.5) (end 153 30.5) (width 0.2) (layer "B.Cu") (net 9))
 (segment (start 154.96 32.46) (end 154.96 83.1485) (width 0.2) (layer "B.Cu") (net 9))
 (segment (start 153 30.5) (end 154.96 32.46) (width 0.2) (layer "B.Cu") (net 9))
 (segment (start 171.5 90) (end 153.5 90) (width 0.2) (layer "B.Cu") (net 8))
 (segment (start 152.42 88.92) (end 152.42 83.1485) (width 0.2) (layer "B.Cu") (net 8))
 (segment (start 153.5 90) (end 152.42 88.92) (width 0.2) (layer "B.Cu") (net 8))
 (segment (start 172.04 66) (end 172.04 89.46) (width 0.2) (layer "B.Cu") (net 8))
 (segment (start 172.04 89.46) (end 171.5 90) (width 0.2) (layer "B.Cu") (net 8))
 (segment (start 103.5 92.5) (end 150 92.5) (width 0.2) (layer "B.Cu") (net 11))
 (segment (start 81 70) (end 103.5 92.5) (width 0.2) (layer "B.Cu") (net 11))
 (segment (start 150 92.5) (end 149.88 92.38) (width 0.2) (layer "B.Cu") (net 11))
 (segment (start 149.88 92.38) (end 149.88 83.1485) (width 0.2) (layer "B.Cu") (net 11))
 (segment (start 139.54 102.5) (end 157.5 102.5) (width 0.2) (layer "B.Cu") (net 6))
 (segment (start 136.54 99.5) (end 139.54 102.5) (width 0.2) (layer "B.Cu") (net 6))
 (segment (start 157.5 102.5) (end 157.5 98.3885) (width 0.2) (layer "B.Cu") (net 6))
 (segment (start 165.74 85.5) (end 165.12 84.88) (width 0.2) (layer "F.Cu") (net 1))
 (segment (start 176 83.5) (end 174 85.5) (width 0.2) (layer "F.Cu") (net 1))
 (segment (start 174 85.5) (end 165.74 85.5) (width 0.2) (layer "F.Cu") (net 1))
 (segment (start 129.08 48.12) (end 171.12 48.12) (width 0.2) (layer "F.Cu") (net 1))
 (segment (start 165.12 84.88) (end 165.12 83.1485) (width 0.2) (layer "F.Cu") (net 1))
 (segment (start 176 53) (end 176 83.5) (width 0.2) (layer "F.Cu") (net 1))
 (segment (start 171.12 48.12) (end 176 53) (width 0.2) (layer "F.Cu") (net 1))
 (segment (start 162.58 90.92) (end 162.58 83.1485) (width 0.2) (layer "F.Cu") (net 4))
 (segment (start 139.5 90.5) (end 140 91) (width 0.2) (layer "F.Cu") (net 4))
 (segment (start 162.5 91) (end 162.58 90.92) (width 0.2) (layer "F.Cu") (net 4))
 (segment (start 140 91) (end 162.5 91) (width 0.2) (layer "F.Cu") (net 4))
 (via (at 139.5 90.5) (size 0.6) (drill 0.3) (layers "F.Cu" "B.Cu") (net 4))
 (segment (start 109.04 67.85) (end 129.35 67.85) (width 0.2) (layer "B.Cu") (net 4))
 (segment (start 138.5 89.5) (end 139.5 90.5) (width 0.2) (layer "B.Cu") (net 4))
 (segment (start 138.5 77) (end 138.5 89.5) (width 0.2) (layer "B.Cu") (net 4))
 (segment (start 129.35 67.85) (end 138.5 77) (width 0.2) (layer "B.Cu") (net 4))
 (segment (start 148.58 67.54) (end 160.04 79) (width 0.2) (layer "F.Cu") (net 10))
 (segment (start 160.04 79) (end 160.04 83.1485) (width 0.2) (layer "F.Cu") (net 10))
 (segment (start 155.46 87.04) (end 157.5 85) (width 0.2) (layer "F.Cu") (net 13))
 (segment (start 128.58 87.04) (end 155.46 87.04) (width 0.2) (layer "F.Cu") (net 13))
 (segment (start 157.5 85) (end 157.5 83.1485) (width 0.2) (layer "F.Cu") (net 13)))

